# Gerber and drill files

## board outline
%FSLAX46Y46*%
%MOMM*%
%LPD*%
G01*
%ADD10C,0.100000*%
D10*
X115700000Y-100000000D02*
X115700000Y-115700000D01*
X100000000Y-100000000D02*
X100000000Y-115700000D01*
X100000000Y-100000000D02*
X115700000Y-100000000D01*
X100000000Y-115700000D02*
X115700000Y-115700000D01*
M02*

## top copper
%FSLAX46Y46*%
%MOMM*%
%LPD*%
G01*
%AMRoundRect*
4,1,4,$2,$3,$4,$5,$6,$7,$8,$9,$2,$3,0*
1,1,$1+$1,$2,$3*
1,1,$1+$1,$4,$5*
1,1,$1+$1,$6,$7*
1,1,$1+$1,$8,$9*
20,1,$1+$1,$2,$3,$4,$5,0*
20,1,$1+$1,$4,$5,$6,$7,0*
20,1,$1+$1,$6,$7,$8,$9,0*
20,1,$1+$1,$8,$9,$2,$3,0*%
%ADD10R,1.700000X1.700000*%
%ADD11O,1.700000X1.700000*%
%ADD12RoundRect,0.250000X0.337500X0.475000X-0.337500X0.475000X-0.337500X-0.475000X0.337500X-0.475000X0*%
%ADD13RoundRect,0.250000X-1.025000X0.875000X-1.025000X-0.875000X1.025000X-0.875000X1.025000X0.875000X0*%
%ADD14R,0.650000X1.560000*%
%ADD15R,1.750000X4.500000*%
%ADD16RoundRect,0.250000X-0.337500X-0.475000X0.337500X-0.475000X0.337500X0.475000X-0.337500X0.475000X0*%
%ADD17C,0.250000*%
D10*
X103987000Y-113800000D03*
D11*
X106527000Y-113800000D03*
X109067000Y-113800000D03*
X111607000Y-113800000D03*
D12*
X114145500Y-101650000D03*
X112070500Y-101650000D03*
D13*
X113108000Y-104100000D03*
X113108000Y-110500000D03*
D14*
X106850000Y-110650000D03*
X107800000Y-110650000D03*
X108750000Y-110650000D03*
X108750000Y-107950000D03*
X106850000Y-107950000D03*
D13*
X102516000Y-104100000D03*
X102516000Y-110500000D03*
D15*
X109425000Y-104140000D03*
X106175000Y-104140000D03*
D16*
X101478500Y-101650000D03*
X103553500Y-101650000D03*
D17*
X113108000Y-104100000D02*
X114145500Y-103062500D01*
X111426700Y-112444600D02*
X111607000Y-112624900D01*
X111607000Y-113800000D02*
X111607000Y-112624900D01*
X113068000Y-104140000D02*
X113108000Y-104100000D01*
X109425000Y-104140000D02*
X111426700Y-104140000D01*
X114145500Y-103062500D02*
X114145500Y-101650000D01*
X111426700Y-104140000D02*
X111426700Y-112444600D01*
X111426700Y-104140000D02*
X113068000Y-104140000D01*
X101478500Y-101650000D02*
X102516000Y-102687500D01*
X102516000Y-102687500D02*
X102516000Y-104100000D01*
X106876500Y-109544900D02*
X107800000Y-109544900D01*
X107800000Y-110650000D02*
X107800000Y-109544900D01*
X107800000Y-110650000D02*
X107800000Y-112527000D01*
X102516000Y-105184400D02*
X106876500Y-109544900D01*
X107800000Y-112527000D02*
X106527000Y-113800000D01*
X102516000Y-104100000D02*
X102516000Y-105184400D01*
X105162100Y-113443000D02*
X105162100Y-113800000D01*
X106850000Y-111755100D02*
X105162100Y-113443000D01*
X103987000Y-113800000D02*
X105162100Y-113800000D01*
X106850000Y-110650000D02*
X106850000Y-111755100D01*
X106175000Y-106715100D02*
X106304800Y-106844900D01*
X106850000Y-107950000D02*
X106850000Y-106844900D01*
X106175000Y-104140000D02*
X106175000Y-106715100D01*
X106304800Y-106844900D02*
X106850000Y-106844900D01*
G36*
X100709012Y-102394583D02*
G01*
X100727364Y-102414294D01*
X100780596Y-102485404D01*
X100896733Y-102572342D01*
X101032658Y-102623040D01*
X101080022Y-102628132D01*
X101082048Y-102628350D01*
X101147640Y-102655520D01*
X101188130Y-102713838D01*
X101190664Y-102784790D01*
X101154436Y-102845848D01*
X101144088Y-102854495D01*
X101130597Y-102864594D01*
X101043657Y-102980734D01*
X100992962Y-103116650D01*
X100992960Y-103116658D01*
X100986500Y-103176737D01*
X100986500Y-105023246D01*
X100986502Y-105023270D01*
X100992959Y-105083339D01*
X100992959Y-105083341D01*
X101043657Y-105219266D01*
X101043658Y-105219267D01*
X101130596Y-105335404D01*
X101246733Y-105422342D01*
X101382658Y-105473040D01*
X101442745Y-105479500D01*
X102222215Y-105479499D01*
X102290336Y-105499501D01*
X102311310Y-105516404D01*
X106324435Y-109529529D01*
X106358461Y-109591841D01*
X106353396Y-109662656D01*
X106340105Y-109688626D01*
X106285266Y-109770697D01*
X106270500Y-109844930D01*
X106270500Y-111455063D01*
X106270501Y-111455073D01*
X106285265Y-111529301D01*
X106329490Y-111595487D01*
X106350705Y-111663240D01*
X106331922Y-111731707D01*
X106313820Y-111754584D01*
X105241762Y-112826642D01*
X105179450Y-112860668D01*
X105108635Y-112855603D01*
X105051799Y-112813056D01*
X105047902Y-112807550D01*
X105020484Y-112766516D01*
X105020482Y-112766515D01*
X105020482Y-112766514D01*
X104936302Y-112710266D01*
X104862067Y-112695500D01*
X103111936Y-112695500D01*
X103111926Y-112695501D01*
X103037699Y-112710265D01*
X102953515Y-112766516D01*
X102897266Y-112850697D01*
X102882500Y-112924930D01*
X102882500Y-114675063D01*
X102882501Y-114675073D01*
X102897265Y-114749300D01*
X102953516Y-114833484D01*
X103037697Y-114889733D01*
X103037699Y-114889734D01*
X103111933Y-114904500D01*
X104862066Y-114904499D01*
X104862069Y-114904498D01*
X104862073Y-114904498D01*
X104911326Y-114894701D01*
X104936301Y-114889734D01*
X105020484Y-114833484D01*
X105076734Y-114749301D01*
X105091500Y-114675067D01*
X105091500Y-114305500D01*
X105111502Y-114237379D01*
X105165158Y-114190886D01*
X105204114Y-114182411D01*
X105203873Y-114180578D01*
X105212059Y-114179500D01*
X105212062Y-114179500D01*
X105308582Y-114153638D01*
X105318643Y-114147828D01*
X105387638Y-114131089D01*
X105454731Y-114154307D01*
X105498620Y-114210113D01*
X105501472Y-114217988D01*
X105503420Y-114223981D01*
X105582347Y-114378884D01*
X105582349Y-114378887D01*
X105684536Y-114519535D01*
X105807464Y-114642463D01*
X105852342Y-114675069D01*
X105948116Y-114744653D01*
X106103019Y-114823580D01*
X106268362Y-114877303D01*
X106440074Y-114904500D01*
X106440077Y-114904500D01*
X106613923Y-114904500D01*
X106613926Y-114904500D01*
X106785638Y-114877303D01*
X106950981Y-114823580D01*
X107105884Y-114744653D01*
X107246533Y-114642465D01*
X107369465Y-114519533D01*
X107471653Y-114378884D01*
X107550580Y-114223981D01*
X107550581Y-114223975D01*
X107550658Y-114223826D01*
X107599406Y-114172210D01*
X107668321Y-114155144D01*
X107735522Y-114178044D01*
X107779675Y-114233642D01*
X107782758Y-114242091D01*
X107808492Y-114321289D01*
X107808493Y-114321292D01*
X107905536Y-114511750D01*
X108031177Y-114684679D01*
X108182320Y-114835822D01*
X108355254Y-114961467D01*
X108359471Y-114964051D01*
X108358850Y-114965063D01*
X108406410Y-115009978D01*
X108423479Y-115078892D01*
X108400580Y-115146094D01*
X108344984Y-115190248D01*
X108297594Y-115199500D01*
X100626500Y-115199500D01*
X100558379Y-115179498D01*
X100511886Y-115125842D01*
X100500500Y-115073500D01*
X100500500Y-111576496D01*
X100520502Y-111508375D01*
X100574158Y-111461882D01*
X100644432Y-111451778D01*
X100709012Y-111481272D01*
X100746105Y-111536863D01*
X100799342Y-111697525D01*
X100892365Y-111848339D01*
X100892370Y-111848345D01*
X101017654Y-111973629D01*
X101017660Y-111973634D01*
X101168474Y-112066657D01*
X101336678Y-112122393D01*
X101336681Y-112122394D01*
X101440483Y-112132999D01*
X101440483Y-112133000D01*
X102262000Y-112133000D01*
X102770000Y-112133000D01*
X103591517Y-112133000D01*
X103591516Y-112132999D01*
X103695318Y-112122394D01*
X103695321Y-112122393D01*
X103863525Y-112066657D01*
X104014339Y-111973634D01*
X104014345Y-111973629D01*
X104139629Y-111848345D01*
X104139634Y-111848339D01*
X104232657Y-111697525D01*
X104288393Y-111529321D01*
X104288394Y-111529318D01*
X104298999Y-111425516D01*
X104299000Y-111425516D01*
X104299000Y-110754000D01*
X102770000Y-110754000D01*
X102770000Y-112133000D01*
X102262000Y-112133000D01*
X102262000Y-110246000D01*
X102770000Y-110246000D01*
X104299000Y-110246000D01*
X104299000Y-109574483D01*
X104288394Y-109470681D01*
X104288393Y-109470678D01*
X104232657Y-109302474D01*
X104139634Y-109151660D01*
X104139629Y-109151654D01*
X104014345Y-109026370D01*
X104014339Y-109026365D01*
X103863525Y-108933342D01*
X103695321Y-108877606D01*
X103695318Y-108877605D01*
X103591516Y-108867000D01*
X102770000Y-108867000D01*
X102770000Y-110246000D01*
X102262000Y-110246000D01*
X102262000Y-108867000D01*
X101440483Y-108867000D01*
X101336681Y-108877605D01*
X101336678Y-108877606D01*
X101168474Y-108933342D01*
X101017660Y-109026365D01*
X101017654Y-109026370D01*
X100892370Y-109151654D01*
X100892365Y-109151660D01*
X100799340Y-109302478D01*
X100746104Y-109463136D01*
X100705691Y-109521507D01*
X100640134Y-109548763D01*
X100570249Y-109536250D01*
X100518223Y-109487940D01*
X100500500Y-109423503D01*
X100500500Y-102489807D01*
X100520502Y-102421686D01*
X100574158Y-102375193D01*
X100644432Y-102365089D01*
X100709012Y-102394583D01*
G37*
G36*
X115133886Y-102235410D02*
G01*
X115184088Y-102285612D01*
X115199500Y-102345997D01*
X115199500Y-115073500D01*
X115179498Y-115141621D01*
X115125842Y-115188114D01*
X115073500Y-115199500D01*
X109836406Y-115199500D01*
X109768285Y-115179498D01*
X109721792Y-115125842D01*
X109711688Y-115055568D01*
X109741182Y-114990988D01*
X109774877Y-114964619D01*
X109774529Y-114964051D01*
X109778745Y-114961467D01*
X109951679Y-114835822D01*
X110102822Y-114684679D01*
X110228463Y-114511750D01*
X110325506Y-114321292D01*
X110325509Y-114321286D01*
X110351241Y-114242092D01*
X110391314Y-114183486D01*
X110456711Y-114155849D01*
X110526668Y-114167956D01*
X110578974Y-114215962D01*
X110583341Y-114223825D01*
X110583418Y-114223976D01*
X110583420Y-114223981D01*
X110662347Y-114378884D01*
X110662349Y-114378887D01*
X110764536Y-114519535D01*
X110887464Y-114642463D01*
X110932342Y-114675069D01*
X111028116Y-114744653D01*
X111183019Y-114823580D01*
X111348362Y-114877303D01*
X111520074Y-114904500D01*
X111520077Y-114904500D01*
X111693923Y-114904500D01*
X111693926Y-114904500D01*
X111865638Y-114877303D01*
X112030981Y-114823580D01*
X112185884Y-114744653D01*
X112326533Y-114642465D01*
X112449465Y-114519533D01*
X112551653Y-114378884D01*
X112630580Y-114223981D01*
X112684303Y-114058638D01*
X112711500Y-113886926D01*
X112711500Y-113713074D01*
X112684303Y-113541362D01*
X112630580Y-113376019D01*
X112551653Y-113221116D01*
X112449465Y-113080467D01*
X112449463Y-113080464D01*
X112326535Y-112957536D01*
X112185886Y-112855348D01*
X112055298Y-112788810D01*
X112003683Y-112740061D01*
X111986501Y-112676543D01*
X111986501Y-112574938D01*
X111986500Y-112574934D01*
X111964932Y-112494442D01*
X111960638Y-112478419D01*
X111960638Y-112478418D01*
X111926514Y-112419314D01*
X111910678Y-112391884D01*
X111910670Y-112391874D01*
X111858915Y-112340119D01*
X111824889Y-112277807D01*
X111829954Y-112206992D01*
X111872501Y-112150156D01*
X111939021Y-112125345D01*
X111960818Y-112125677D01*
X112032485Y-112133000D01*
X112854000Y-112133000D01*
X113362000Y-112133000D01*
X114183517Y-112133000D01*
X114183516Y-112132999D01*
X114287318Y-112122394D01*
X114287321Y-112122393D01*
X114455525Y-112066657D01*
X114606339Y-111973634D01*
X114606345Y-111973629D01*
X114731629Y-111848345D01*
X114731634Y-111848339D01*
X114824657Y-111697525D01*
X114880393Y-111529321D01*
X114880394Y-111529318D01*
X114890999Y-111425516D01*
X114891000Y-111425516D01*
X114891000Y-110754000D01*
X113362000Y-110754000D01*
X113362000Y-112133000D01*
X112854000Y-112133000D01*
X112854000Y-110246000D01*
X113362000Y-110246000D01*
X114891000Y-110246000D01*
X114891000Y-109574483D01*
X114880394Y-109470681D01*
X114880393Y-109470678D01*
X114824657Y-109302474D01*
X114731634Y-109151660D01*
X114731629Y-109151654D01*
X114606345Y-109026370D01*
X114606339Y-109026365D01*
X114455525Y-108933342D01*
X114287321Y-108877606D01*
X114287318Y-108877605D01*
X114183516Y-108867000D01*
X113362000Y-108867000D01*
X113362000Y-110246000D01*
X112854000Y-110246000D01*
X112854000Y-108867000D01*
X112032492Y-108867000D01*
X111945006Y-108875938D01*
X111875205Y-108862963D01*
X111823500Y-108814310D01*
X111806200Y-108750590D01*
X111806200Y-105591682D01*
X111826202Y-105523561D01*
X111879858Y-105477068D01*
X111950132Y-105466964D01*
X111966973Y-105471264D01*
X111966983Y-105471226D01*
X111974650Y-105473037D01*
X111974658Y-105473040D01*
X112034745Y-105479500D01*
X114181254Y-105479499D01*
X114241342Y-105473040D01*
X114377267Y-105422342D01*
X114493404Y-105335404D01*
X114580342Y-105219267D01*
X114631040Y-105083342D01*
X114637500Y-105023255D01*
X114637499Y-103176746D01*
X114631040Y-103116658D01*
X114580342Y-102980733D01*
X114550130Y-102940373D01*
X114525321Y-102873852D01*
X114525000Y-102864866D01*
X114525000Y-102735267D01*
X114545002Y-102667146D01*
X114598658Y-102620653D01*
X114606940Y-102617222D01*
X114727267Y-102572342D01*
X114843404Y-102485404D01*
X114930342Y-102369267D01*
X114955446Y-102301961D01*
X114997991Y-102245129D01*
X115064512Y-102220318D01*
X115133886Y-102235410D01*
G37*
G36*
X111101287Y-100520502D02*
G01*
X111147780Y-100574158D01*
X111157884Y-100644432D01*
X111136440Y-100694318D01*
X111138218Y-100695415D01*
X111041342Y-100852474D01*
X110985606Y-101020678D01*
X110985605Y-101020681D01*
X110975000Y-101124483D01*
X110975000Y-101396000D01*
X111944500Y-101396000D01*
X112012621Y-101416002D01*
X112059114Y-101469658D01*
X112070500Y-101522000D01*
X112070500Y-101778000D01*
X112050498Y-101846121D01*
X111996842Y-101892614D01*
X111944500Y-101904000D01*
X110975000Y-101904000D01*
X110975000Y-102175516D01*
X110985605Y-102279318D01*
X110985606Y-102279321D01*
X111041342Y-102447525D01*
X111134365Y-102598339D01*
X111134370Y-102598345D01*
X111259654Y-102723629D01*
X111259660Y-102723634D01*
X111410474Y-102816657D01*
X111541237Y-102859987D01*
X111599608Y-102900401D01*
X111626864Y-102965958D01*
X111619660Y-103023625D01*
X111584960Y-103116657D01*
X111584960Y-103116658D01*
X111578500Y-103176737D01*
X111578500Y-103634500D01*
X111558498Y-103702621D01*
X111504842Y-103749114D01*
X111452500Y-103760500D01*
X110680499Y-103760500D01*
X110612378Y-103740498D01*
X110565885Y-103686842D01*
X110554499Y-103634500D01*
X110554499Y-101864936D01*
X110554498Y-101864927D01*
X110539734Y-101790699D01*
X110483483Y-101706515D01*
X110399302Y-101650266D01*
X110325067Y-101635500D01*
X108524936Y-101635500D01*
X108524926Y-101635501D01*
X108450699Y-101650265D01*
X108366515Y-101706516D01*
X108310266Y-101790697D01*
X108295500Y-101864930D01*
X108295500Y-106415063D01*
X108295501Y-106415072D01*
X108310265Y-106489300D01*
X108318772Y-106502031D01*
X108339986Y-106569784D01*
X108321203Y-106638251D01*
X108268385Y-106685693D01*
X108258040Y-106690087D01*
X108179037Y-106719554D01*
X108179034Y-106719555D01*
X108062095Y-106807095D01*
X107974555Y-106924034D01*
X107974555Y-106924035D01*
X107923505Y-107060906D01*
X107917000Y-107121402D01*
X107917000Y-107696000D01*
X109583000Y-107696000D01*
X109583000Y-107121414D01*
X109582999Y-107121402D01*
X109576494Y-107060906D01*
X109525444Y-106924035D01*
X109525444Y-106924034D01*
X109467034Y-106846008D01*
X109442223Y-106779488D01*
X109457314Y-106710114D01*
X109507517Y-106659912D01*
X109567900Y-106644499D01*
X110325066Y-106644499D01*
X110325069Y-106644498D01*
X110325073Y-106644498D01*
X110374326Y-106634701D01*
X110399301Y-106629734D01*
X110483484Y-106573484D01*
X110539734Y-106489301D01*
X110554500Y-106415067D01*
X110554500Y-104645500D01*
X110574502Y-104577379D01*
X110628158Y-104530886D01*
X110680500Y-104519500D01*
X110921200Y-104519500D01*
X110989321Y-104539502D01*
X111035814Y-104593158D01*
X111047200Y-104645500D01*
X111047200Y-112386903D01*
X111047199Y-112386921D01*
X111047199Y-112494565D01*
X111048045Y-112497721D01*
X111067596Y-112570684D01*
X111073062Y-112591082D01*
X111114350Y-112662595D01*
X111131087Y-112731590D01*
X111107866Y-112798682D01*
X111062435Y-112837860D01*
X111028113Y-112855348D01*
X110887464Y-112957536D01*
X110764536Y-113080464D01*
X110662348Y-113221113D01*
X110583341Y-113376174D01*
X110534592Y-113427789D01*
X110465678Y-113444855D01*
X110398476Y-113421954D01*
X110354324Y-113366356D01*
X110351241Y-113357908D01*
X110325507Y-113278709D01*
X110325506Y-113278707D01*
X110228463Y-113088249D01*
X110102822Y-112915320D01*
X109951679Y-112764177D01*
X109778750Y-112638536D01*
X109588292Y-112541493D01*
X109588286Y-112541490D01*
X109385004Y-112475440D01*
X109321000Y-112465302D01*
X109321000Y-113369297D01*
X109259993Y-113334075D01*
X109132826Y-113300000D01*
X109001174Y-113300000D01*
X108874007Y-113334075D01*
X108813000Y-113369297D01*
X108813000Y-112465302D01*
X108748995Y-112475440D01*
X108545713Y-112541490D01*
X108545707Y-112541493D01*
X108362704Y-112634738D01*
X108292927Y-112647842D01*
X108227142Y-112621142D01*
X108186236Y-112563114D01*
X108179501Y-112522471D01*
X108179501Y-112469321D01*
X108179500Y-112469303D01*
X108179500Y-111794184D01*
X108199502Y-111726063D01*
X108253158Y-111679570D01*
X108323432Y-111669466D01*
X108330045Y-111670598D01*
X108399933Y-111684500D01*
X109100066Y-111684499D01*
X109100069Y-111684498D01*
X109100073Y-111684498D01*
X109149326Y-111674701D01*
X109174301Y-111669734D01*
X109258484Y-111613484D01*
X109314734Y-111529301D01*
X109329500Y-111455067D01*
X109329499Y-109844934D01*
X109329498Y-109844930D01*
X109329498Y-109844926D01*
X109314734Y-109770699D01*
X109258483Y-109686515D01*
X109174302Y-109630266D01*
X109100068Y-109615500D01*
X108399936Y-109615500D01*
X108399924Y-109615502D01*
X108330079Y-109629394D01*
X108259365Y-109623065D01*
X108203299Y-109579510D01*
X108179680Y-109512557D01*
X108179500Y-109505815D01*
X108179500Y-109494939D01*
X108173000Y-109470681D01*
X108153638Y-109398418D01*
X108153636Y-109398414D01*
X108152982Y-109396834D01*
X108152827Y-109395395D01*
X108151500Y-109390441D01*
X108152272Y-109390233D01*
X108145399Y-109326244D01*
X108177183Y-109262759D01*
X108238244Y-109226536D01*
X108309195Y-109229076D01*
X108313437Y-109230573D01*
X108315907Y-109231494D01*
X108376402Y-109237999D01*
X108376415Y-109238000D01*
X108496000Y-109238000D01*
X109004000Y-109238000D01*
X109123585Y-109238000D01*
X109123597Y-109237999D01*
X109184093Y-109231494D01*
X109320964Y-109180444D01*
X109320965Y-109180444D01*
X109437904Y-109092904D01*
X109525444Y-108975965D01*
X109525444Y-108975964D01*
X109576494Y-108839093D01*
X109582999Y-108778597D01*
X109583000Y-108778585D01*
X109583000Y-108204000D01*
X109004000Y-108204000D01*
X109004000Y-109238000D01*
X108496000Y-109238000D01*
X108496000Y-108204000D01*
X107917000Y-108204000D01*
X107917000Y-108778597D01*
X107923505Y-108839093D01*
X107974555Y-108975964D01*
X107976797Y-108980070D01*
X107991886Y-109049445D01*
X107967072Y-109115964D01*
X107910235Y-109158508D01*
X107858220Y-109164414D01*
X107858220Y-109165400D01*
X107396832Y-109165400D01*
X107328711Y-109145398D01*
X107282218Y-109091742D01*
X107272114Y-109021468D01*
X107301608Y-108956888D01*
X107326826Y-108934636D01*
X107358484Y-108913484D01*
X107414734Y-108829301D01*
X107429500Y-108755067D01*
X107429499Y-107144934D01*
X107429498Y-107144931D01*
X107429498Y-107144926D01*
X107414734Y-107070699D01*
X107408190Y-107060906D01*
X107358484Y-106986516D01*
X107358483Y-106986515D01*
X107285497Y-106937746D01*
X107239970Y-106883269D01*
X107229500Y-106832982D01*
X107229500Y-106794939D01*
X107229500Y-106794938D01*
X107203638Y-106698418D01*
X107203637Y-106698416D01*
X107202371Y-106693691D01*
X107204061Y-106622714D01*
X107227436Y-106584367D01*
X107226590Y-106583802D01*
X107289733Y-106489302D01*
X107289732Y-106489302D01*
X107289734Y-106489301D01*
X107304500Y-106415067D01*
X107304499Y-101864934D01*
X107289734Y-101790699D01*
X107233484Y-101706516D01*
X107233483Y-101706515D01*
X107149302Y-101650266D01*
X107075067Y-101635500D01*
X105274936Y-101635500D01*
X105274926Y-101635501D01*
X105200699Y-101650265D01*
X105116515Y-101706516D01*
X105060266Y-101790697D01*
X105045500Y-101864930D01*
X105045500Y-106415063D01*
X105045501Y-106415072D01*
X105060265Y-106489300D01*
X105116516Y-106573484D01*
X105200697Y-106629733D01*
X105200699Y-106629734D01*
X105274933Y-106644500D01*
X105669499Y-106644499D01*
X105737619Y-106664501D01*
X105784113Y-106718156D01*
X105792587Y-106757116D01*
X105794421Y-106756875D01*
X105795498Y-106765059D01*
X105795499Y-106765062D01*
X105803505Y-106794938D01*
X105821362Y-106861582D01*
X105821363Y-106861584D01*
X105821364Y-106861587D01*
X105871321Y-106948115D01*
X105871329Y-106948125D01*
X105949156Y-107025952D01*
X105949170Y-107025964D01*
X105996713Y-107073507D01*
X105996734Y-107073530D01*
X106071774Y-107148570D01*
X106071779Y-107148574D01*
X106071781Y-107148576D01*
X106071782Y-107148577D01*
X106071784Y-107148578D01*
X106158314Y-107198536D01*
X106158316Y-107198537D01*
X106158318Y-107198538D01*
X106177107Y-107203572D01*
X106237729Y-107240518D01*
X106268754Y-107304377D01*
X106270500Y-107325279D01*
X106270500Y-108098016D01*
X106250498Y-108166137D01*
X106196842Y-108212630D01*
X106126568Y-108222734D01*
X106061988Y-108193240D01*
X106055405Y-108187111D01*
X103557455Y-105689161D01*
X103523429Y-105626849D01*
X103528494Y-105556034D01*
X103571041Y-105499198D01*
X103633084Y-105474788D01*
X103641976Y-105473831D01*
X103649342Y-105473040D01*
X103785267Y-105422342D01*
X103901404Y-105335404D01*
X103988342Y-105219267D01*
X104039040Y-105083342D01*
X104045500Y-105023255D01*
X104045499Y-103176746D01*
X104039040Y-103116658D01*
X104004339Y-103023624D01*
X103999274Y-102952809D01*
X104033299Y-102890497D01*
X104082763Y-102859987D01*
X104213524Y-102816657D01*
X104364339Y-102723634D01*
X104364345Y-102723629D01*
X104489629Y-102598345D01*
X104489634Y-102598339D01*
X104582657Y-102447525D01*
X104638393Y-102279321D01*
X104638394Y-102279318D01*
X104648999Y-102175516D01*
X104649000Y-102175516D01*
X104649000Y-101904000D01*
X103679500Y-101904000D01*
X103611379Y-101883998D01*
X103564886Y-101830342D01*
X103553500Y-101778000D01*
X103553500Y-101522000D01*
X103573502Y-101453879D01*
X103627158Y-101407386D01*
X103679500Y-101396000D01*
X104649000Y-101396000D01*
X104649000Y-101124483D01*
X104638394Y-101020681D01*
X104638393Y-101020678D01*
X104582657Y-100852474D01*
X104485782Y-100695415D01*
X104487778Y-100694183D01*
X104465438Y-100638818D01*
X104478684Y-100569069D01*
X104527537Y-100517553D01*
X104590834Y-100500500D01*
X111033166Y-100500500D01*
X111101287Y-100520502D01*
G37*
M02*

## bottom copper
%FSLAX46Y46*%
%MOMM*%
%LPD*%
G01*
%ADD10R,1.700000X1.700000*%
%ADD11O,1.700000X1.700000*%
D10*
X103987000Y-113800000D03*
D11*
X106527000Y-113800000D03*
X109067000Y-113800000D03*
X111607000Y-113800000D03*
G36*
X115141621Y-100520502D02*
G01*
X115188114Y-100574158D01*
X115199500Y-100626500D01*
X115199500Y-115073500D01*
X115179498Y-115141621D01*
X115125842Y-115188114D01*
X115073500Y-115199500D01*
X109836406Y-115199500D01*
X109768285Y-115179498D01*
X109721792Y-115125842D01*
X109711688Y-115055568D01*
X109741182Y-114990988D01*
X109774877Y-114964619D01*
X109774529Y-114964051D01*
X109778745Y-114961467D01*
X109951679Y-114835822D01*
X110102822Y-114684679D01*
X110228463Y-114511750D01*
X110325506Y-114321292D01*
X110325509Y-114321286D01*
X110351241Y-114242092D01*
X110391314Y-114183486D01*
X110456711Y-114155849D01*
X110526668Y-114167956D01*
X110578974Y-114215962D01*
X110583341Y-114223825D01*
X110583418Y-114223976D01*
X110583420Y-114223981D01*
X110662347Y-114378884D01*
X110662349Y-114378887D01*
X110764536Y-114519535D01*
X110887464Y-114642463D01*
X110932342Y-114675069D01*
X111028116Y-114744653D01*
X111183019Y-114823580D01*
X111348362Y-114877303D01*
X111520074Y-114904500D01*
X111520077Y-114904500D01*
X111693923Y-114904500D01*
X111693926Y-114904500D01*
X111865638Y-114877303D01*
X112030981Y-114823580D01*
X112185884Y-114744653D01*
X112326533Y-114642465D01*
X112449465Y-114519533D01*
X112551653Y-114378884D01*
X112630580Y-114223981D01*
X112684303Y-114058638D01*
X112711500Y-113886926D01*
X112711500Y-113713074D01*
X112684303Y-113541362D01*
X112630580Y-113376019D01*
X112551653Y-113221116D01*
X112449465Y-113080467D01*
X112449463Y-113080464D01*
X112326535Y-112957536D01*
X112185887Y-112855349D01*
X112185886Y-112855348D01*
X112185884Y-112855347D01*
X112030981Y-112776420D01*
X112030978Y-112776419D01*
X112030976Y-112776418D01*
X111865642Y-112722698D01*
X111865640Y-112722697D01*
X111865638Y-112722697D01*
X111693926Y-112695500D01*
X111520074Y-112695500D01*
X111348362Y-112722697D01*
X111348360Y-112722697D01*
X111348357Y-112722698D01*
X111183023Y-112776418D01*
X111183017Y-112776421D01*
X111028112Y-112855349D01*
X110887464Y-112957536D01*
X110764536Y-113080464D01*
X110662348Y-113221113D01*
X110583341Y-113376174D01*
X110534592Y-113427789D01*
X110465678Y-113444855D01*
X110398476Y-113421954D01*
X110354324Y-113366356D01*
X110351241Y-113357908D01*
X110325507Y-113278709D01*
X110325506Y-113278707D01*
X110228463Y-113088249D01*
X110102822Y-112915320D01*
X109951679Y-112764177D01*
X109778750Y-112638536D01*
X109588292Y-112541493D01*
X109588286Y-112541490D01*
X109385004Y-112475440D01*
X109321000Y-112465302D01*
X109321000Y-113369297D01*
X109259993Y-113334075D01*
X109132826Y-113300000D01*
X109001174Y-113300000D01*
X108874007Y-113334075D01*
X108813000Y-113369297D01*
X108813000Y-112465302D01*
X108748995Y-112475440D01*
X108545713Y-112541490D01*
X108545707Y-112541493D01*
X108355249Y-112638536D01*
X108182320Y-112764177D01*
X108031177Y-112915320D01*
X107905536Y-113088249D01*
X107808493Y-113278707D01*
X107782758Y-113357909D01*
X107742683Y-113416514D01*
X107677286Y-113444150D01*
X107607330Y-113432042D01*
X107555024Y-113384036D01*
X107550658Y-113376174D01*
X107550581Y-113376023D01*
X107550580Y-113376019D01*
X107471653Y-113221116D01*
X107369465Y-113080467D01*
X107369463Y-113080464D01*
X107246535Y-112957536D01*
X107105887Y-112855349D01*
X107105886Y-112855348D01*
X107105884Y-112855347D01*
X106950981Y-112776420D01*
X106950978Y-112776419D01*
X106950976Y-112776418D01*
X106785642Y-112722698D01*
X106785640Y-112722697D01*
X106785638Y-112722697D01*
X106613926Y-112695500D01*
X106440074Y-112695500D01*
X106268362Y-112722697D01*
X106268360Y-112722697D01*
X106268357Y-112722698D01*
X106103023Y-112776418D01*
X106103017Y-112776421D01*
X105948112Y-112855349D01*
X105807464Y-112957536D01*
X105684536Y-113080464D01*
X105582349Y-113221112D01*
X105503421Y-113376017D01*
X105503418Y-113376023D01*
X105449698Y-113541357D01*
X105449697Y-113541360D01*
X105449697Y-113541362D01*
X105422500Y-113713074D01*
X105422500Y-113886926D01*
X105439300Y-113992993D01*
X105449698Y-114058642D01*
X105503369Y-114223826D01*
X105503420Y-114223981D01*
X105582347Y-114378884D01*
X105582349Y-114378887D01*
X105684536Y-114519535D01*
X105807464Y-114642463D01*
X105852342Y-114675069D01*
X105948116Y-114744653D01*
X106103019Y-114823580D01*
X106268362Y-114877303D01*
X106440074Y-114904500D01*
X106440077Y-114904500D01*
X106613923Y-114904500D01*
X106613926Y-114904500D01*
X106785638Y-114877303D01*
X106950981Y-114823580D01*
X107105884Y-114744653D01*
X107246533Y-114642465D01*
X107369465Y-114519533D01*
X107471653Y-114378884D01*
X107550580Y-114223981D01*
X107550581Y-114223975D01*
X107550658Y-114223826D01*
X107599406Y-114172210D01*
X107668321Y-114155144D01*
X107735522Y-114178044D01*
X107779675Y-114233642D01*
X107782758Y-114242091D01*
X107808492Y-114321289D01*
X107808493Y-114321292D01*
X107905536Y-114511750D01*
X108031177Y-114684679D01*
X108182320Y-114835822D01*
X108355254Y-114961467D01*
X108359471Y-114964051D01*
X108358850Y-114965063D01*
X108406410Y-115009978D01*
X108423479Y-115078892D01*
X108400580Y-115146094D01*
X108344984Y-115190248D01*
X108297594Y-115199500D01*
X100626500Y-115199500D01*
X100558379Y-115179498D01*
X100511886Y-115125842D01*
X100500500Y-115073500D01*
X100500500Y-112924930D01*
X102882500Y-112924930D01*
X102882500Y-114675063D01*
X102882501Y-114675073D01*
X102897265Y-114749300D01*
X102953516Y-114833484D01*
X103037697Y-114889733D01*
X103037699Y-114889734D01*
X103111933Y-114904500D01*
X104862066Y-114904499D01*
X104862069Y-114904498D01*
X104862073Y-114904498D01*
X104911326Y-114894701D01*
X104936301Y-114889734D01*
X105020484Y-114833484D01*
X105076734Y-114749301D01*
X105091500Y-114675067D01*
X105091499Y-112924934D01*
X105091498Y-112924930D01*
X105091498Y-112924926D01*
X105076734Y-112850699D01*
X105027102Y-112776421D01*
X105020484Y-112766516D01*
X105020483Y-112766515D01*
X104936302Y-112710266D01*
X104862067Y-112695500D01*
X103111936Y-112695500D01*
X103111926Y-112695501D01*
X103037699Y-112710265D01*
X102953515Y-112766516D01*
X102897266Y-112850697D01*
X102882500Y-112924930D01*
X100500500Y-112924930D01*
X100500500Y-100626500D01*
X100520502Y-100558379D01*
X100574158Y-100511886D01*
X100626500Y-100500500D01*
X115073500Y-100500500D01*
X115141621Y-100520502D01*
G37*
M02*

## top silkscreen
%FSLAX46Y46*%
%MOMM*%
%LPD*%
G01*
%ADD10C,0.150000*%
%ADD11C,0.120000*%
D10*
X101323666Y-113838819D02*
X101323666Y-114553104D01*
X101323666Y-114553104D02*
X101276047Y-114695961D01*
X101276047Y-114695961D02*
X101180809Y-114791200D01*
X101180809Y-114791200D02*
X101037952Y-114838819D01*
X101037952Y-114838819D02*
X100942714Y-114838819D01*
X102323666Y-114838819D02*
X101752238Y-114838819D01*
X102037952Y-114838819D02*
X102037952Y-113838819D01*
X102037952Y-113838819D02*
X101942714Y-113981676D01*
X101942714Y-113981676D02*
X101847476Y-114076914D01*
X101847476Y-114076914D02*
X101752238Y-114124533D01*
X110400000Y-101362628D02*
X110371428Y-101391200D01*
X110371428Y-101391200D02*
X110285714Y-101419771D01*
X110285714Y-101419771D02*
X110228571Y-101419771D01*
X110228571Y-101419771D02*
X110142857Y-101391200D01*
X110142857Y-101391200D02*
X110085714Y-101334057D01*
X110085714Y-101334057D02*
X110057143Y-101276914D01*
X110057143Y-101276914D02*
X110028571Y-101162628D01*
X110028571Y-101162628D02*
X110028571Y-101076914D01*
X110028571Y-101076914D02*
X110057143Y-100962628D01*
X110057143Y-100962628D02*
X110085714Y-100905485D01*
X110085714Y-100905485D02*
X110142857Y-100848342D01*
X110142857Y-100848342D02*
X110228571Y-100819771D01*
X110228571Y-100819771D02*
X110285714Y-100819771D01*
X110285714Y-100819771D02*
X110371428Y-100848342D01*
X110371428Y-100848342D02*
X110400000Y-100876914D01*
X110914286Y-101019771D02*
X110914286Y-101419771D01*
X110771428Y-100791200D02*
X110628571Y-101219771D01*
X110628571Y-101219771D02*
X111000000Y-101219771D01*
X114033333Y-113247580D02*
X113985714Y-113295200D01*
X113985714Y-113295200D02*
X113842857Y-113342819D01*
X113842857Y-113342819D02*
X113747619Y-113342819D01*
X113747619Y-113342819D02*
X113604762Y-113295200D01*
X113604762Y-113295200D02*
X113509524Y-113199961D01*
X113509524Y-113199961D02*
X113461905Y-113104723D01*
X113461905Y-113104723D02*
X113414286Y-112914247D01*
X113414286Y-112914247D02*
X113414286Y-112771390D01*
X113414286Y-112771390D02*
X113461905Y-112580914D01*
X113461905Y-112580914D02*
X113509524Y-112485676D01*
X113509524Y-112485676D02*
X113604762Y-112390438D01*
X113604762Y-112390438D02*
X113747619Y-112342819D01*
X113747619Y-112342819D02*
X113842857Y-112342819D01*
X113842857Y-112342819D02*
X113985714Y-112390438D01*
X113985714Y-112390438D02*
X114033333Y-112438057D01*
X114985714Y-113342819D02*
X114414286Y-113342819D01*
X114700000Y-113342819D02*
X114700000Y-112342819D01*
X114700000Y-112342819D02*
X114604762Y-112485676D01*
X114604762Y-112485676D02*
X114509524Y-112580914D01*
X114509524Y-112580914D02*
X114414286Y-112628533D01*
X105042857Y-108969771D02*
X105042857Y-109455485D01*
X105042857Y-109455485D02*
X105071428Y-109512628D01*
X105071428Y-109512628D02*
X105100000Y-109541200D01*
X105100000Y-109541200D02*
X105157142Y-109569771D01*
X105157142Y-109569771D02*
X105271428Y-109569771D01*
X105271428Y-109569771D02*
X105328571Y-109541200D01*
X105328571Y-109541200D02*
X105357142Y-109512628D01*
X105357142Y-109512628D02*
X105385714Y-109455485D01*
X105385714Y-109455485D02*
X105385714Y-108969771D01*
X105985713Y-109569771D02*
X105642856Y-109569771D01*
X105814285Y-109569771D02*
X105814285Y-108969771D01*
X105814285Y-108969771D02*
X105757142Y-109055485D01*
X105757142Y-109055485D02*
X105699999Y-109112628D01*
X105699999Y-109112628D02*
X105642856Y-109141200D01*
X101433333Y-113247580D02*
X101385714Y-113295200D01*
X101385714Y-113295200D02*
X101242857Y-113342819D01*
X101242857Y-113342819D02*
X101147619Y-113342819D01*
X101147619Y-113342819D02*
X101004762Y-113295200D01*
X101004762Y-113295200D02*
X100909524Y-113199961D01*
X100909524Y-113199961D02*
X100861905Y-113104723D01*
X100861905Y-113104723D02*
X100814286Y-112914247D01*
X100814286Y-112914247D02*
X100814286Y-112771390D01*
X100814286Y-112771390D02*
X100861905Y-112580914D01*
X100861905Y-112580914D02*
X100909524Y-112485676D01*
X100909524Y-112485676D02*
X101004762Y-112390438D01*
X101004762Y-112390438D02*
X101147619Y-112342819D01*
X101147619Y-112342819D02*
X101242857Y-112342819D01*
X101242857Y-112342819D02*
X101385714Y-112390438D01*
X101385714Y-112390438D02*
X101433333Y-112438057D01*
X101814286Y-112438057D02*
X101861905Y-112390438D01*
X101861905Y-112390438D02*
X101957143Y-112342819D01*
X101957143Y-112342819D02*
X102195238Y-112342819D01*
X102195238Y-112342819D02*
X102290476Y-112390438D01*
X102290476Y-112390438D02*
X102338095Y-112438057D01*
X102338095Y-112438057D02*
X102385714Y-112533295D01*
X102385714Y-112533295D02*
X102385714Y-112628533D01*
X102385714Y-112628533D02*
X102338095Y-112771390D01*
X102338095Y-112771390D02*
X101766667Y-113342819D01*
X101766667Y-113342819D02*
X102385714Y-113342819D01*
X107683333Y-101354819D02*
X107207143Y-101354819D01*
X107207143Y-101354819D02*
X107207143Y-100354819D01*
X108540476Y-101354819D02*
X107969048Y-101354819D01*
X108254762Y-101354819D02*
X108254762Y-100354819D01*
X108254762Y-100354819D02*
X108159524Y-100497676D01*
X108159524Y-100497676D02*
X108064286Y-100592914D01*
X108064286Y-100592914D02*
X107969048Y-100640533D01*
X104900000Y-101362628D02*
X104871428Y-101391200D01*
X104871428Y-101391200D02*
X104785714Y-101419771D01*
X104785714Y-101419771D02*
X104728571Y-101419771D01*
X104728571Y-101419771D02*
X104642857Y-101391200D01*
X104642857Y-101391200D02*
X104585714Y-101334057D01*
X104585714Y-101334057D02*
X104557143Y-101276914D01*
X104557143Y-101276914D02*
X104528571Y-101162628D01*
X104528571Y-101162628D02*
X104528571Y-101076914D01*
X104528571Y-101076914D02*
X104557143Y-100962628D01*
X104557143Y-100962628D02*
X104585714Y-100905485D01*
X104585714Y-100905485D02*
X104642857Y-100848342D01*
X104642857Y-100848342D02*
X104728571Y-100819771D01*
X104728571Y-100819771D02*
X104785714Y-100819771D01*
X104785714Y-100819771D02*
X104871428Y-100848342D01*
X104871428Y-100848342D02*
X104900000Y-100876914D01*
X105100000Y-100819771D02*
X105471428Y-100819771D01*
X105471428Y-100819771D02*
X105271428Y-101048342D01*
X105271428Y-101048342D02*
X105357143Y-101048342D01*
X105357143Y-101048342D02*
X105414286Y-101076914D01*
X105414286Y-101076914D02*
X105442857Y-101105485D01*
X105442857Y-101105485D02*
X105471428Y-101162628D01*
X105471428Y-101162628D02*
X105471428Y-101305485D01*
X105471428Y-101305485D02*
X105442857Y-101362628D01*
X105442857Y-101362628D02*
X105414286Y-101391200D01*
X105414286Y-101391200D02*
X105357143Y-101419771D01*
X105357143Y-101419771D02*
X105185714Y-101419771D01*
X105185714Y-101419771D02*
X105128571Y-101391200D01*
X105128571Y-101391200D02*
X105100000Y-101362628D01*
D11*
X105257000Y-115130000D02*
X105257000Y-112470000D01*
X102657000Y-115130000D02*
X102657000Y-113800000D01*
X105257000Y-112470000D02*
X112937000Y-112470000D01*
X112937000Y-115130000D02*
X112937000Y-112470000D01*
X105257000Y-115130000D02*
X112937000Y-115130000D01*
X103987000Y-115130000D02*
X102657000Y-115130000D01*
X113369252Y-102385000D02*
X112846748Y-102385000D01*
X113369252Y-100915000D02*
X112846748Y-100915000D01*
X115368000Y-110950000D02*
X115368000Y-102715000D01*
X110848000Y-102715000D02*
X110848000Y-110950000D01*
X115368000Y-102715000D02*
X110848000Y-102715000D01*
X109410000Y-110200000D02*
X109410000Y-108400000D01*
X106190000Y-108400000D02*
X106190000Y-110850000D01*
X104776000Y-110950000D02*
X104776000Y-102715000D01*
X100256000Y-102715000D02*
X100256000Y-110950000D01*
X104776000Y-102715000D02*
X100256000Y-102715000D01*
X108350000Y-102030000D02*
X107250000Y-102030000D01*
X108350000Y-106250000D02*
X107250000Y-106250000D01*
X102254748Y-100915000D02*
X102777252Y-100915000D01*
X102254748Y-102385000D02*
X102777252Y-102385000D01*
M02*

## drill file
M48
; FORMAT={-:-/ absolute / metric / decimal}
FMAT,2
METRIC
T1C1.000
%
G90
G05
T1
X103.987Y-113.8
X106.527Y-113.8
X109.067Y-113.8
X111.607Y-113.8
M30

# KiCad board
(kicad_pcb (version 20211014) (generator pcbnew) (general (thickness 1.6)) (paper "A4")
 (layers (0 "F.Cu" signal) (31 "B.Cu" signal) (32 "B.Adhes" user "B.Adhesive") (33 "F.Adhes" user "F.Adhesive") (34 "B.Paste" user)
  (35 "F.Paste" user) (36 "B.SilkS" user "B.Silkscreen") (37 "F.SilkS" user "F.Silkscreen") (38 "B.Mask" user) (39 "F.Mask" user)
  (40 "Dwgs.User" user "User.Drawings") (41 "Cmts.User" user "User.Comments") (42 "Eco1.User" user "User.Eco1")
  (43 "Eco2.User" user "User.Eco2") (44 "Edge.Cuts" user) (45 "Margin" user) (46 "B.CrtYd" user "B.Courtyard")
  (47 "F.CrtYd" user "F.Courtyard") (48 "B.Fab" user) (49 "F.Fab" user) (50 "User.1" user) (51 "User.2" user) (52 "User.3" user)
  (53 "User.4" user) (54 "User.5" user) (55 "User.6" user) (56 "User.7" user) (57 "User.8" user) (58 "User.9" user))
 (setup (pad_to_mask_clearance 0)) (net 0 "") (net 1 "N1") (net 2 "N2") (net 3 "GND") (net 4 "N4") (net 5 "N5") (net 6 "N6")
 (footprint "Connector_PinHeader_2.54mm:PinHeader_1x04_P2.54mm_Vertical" (layer "F.Cu") (at 103.987 113.8 90)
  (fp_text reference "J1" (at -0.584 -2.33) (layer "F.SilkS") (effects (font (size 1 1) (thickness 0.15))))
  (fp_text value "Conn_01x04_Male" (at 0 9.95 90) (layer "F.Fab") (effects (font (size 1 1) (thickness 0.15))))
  (fp_line (start -1.33 1.27) (end 1.33 1.27) (layer "F.SilkS") (width 0.12))
  (fp_line (start -1.33 -1.33) (end 0 -1.33) (layer "F.SilkS") (width 0.12))
  (fp_line (start 1.33 1.27) (end 1.33 8.95) (layer "F.SilkS") (width 0.12))
  (fp_line (start -1.33 8.95) (end 1.33 8.95) (layer "F.SilkS") (width 0.12))
  (fp_line (start -1.33 1.27) (end -1.33 8.95) (layer "F.SilkS") (width 0.12))
  (fp_line (start -1.33 0) (end -1.33 -1.33) (layer "F.SilkS") (width 0.12))
  (pad "1" thru_hole rect (at 0 0 90) (size 1.7 1.7) (drill 1) (layers *.Cu *.Mask) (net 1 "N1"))
  (pad "2" thru_hole oval (at 0 2.54 90) (size 1.7 1.7) (drill 1) (layers *.Cu *.Mask) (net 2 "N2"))
  (pad "3" thru_hole oval (at 0 5.08 90) (size 1.7 1.7) (drill 1) (layers *.Cu *.Mask) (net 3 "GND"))
  (pad "4" thru_hole oval (at 0 7.62 90) (size 1.7 1.7) (drill 1) (layers *.Cu *.Mask) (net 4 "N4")))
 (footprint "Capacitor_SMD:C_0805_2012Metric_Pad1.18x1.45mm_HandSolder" (layer "F.Cu") (at 113.108 101.65 180)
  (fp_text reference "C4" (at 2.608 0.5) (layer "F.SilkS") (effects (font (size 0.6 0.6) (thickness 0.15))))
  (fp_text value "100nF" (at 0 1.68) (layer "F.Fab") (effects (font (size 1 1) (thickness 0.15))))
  (fp_line (start -0.261252 -0.735) (end 0.261252 -0.735) (layer "F.SilkS") (width 0.12))
  (fp_line (start -0.261252 0.735) (end 0.261252 0.735) (layer "F.SilkS") (width 0.12))
  (pad "1" smd roundrect (at -1.0375 0 180) (size 1.175 1.45) (layers "F.Cu" "F.Paste" "F.Mask") (roundrect_rratio 0.2127659574)
   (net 4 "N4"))
  (pad "2" smd roundrect (at 1.0375 0 180) (size 1.175 1.45) (layers "F.Cu" "F.Paste" "F.Mask") (roundrect_rratio 0.2127659574)
   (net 3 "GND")))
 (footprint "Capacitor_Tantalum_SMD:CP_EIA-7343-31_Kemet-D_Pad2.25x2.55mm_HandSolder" (layer "F.Cu") (at 113.108 107.3 -90)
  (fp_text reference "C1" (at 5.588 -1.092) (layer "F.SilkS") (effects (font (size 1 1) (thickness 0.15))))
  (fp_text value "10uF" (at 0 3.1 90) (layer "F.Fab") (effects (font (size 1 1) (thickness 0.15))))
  (fp_line (start 3.65 -2.26) (end -4.585 -2.26) (layer "F.SilkS") (width 0.12))
  (fp_line (start -4.585 2.26) (end 3.65 2.26) (layer "F.SilkS") (width 0.12))
  (fp_line (start -4.585 -2.26) (end -4.585 2.26) (layer "F.SilkS") (width 0.12))
  (pad "1" smd roundrect (at -3.2 0 270) (size 2.25 2.55) (layers "F.Cu" "F.Paste" "F.Mask") (roundrect_rratio 0.1111111111) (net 4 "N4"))
  (pad "2" smd roundrect (at 3.2 0 270) (size 2.25 2.55) (layers "F.Cu" "F.Paste" "F.Mask") (roundrect_rratio 0.1111111111) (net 3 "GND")))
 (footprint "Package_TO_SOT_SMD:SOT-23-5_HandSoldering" (layer "F.Cu") (at 107.8 109.3 90)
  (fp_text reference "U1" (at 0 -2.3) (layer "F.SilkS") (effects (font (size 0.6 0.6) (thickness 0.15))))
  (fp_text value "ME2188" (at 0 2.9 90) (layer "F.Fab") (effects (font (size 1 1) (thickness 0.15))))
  (fp_line (start -0.9 1.61) (end 0.9 1.61) (layer "F.SilkS") (width 0.12))
  (fp_line (start 0.9 -1.61) (end -1.55 -1.61) (layer "F.SilkS") (width 0.12))
  (pad "1" smd rect (at -1.35 -0.95 90) (size 1.56 0.65) (layers "F.Cu" "F.Paste" "F.Mask") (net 1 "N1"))
  (pad "2" smd rect (at -1.35 0 90) (size 1.56 0.65) (layers "F.Cu" "F.Paste" "F.Mask") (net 2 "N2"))
  (pad "3" smd rect (at -1.35 0.95 90) (size 1.56 0.65) (layers "F.Cu" "F.Paste" "F.Mask") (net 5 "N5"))
  (pad "4" smd rect (at 1.35 0.95 90) (size 1.56 0.65) (layers "F.Cu" "F.Paste" "F.Mask") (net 3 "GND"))
  (pad "5" smd rect (at 1.35 -0.95 90) (size 1.56 0.65) (layers "F.Cu" "F.Paste" "F.Mask") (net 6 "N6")))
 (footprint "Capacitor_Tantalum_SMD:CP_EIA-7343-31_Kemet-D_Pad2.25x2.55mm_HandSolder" (layer "F.Cu") (at 102.516 107.3 -90)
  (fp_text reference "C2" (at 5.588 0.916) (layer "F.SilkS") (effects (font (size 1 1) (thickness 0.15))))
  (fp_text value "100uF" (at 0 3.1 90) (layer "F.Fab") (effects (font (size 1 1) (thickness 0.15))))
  (fp_line (start 3.65 -2.26) (end -4.585 -2.26) (layer "F.SilkS") (width 0.12))
  (fp_line (start -4.585 2.26) (end 3.65 2.26) (layer "F.SilkS") (width 0.12))
  (fp_line (start -4.585 -2.26) (end -4.585 2.26) (layer "F.SilkS") (width 0.12))
  (pad "1" smd roundrect (at -3.2 0 270) (size 2.25 2.55) (layers "F.Cu" "F.Paste" "F.Mask") (roundrect_rratio 0.1111111111) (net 2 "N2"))
  (pad "2" smd roundrect (at 3.2 0 270) (size 2.25 2.55) (layers "F.Cu" "F.Paste" "F.Mask") (roundrect_rratio 0.1111111111) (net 3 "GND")))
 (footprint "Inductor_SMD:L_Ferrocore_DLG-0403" (layer "F.Cu") (at 107.8 104.14 180)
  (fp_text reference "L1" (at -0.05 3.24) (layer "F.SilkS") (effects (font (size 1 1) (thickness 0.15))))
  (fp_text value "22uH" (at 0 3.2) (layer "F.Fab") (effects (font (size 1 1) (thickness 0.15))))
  (fp_line (start -0.55 2.11) (end 0.55 2.11) (layer "F.SilkS") (width 0.12))
  (fp_line (start -0.55 -2.11) (end 0.55 -2.11) (layer "F.SilkS") (width 0.12))
  (pad "1" smd rect (at -1.625 0 180) (size 1.75 4.5) (layers "F.Cu" "F.Paste" "F.Mask") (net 4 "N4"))
  (pad "2" smd rect (at 1.625 0 180) (size 1.75 4.5) (layers "F.Cu" "F.Paste" "F.Mask") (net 6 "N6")))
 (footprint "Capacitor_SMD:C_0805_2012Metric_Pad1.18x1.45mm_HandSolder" (layer "F.Cu") (at 102.516 101.65)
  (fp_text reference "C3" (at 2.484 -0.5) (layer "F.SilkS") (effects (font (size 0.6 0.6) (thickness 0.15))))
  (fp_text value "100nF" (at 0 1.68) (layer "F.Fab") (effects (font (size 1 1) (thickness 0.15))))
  (fp_line (start -0.261252 -0.735) (end 0.261252 -0.735) (layer "F.SilkS") (width 0.12))
  (fp_line (start -0.261252 0.735) (end 0.261252 0.735) (layer "F.SilkS") (width 0.12))
  (pad "1" smd roundrect (at -1.0375 0) (size 1.175 1.45) (layers "F.Cu" "F.Paste" "F.Mask") (roundrect_rratio 0.2127659574) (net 2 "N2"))
  (pad "2" smd roundrect (at 1.0375 0) (size 1.175 1.45) (layers "F.Cu" "F.Paste" "F.Mask") (roundrect_rratio 0.2127659574) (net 3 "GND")))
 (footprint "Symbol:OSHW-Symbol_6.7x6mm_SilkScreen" (layer "B.Cu") (at 111.76 104.14 90)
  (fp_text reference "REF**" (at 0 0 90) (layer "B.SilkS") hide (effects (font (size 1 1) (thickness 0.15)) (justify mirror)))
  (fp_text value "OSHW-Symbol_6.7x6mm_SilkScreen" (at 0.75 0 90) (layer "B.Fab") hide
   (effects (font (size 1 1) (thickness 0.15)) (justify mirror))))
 (gr_line (start 115.7 100) (end 115.7 115.7) (layer "Edge.Cuts") (width 0.1))
 (gr_line (start 100 100) (end 100 115.7) (layer "Edge.Cuts") (width 0.1))
 (gr_line (start 100 100) (end 115.7 100) (layer "Edge.Cuts") (width 0.1))
 (gr_line (start 100 115.7) (end 115.7 115.7) (layer "Edge.Cuts") (width 0.1))
 (segment (start 113.108 104.1) (end 114.1455 103.0625) (width 0.25) (layer "F.Cu") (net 4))
 (segment (start 111.4267 112.4446) (end 111.607 112.6249) (width 0.25) (layer "F.Cu") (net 4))
 (segment (start 111.607 113.8) (end 111.607 112.6249) (width 0.25) (layer "F.Cu") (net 4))
 (segment (start 113.068 104.14) (end 113.108 104.1) (width 0.25) (layer "F.Cu") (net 4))
 (segment (start 109.425 104.14) (end 111.4267 104.14) (width 0.25) (layer "F.Cu") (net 4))
 (segment (start 114.1455 103.0625) (end 114.1455 101.65) (width 0.25) (layer "F.Cu") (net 4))
 (segment (start 111.4267 104.14) (end 111.4267 112.4446) (width 0.25) (layer "F.Cu") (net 4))
 (segment (start 111.4267 104.14) (end 113.068 104.14) (width 0.25) (layer "F.Cu") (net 4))
 (segment (start 101.4785 101.65) (end 102.516 102.6875) (width 0.25) (layer "F.Cu") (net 2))
 (segment (start 102.516 102.6875) (end 102.516 104.1) (width 0.25) (layer "F.Cu") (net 2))
 (segment (start 106.8765 109.5449) (end 107.8 109.5449) (width 0.25) (layer "F.Cu") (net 2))
 (segment (start 107.8 110.65) (end 107.8 109.5449) (width 0.25) (layer "F.Cu") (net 2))
 (segment (start 107.8 110.65) (end 107.8 112.527) (width 0.25) (layer "F.Cu") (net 2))
 (segment (start 102.516 105.1844) (end 106.8765 109.5449) (width 0.25) (layer "F.Cu") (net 2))
 (segment (start 107.8 112.527) (end 106.527 113.8) (width 0.25) (layer "F.Cu") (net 2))
 (segment (start 102.516 104.1) (end 102.516 105.1844) (width 0.25) (layer "F.Cu") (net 2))
 (segment (start 105.1621 113.443) (end 105.1621 113.8) (width 0.25) (layer "F.Cu") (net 1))
 (segment (start 106.85 111.7551) (end 105.1621 113.443) (width 0.25) (layer "F.Cu") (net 1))
 (segment (start 103.987 113.8) (end 105.1621 113.8) (width 0.25) (layer "F.Cu") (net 1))
 (segment (start 106.85 110.65) (end 106.85 111.7551) (width 0.25) (layer "F.Cu") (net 1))
 (segment (start 106.175 106.7151) (end 106.3048 106.8449) (width 0.25) (layer "F.Cu") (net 6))
 (segment (start 106.85 107.95) (end 106.85 106.8449) (width 0.25) (layer "F.Cu") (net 6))
 (segment (start 106.175 104.14) (end 106.175 106.7151) (width 0.25) (layer "F.Cu") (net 6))
 (segment (start 106.3048 106.8449) (end 106.85 106.8449) (width 0.25) (layer "F.Cu") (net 6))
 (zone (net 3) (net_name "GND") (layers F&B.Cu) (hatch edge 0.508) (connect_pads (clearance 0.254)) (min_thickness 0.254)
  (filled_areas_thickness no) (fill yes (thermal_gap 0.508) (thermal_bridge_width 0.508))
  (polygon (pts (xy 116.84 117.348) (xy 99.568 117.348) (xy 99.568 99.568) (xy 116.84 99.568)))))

